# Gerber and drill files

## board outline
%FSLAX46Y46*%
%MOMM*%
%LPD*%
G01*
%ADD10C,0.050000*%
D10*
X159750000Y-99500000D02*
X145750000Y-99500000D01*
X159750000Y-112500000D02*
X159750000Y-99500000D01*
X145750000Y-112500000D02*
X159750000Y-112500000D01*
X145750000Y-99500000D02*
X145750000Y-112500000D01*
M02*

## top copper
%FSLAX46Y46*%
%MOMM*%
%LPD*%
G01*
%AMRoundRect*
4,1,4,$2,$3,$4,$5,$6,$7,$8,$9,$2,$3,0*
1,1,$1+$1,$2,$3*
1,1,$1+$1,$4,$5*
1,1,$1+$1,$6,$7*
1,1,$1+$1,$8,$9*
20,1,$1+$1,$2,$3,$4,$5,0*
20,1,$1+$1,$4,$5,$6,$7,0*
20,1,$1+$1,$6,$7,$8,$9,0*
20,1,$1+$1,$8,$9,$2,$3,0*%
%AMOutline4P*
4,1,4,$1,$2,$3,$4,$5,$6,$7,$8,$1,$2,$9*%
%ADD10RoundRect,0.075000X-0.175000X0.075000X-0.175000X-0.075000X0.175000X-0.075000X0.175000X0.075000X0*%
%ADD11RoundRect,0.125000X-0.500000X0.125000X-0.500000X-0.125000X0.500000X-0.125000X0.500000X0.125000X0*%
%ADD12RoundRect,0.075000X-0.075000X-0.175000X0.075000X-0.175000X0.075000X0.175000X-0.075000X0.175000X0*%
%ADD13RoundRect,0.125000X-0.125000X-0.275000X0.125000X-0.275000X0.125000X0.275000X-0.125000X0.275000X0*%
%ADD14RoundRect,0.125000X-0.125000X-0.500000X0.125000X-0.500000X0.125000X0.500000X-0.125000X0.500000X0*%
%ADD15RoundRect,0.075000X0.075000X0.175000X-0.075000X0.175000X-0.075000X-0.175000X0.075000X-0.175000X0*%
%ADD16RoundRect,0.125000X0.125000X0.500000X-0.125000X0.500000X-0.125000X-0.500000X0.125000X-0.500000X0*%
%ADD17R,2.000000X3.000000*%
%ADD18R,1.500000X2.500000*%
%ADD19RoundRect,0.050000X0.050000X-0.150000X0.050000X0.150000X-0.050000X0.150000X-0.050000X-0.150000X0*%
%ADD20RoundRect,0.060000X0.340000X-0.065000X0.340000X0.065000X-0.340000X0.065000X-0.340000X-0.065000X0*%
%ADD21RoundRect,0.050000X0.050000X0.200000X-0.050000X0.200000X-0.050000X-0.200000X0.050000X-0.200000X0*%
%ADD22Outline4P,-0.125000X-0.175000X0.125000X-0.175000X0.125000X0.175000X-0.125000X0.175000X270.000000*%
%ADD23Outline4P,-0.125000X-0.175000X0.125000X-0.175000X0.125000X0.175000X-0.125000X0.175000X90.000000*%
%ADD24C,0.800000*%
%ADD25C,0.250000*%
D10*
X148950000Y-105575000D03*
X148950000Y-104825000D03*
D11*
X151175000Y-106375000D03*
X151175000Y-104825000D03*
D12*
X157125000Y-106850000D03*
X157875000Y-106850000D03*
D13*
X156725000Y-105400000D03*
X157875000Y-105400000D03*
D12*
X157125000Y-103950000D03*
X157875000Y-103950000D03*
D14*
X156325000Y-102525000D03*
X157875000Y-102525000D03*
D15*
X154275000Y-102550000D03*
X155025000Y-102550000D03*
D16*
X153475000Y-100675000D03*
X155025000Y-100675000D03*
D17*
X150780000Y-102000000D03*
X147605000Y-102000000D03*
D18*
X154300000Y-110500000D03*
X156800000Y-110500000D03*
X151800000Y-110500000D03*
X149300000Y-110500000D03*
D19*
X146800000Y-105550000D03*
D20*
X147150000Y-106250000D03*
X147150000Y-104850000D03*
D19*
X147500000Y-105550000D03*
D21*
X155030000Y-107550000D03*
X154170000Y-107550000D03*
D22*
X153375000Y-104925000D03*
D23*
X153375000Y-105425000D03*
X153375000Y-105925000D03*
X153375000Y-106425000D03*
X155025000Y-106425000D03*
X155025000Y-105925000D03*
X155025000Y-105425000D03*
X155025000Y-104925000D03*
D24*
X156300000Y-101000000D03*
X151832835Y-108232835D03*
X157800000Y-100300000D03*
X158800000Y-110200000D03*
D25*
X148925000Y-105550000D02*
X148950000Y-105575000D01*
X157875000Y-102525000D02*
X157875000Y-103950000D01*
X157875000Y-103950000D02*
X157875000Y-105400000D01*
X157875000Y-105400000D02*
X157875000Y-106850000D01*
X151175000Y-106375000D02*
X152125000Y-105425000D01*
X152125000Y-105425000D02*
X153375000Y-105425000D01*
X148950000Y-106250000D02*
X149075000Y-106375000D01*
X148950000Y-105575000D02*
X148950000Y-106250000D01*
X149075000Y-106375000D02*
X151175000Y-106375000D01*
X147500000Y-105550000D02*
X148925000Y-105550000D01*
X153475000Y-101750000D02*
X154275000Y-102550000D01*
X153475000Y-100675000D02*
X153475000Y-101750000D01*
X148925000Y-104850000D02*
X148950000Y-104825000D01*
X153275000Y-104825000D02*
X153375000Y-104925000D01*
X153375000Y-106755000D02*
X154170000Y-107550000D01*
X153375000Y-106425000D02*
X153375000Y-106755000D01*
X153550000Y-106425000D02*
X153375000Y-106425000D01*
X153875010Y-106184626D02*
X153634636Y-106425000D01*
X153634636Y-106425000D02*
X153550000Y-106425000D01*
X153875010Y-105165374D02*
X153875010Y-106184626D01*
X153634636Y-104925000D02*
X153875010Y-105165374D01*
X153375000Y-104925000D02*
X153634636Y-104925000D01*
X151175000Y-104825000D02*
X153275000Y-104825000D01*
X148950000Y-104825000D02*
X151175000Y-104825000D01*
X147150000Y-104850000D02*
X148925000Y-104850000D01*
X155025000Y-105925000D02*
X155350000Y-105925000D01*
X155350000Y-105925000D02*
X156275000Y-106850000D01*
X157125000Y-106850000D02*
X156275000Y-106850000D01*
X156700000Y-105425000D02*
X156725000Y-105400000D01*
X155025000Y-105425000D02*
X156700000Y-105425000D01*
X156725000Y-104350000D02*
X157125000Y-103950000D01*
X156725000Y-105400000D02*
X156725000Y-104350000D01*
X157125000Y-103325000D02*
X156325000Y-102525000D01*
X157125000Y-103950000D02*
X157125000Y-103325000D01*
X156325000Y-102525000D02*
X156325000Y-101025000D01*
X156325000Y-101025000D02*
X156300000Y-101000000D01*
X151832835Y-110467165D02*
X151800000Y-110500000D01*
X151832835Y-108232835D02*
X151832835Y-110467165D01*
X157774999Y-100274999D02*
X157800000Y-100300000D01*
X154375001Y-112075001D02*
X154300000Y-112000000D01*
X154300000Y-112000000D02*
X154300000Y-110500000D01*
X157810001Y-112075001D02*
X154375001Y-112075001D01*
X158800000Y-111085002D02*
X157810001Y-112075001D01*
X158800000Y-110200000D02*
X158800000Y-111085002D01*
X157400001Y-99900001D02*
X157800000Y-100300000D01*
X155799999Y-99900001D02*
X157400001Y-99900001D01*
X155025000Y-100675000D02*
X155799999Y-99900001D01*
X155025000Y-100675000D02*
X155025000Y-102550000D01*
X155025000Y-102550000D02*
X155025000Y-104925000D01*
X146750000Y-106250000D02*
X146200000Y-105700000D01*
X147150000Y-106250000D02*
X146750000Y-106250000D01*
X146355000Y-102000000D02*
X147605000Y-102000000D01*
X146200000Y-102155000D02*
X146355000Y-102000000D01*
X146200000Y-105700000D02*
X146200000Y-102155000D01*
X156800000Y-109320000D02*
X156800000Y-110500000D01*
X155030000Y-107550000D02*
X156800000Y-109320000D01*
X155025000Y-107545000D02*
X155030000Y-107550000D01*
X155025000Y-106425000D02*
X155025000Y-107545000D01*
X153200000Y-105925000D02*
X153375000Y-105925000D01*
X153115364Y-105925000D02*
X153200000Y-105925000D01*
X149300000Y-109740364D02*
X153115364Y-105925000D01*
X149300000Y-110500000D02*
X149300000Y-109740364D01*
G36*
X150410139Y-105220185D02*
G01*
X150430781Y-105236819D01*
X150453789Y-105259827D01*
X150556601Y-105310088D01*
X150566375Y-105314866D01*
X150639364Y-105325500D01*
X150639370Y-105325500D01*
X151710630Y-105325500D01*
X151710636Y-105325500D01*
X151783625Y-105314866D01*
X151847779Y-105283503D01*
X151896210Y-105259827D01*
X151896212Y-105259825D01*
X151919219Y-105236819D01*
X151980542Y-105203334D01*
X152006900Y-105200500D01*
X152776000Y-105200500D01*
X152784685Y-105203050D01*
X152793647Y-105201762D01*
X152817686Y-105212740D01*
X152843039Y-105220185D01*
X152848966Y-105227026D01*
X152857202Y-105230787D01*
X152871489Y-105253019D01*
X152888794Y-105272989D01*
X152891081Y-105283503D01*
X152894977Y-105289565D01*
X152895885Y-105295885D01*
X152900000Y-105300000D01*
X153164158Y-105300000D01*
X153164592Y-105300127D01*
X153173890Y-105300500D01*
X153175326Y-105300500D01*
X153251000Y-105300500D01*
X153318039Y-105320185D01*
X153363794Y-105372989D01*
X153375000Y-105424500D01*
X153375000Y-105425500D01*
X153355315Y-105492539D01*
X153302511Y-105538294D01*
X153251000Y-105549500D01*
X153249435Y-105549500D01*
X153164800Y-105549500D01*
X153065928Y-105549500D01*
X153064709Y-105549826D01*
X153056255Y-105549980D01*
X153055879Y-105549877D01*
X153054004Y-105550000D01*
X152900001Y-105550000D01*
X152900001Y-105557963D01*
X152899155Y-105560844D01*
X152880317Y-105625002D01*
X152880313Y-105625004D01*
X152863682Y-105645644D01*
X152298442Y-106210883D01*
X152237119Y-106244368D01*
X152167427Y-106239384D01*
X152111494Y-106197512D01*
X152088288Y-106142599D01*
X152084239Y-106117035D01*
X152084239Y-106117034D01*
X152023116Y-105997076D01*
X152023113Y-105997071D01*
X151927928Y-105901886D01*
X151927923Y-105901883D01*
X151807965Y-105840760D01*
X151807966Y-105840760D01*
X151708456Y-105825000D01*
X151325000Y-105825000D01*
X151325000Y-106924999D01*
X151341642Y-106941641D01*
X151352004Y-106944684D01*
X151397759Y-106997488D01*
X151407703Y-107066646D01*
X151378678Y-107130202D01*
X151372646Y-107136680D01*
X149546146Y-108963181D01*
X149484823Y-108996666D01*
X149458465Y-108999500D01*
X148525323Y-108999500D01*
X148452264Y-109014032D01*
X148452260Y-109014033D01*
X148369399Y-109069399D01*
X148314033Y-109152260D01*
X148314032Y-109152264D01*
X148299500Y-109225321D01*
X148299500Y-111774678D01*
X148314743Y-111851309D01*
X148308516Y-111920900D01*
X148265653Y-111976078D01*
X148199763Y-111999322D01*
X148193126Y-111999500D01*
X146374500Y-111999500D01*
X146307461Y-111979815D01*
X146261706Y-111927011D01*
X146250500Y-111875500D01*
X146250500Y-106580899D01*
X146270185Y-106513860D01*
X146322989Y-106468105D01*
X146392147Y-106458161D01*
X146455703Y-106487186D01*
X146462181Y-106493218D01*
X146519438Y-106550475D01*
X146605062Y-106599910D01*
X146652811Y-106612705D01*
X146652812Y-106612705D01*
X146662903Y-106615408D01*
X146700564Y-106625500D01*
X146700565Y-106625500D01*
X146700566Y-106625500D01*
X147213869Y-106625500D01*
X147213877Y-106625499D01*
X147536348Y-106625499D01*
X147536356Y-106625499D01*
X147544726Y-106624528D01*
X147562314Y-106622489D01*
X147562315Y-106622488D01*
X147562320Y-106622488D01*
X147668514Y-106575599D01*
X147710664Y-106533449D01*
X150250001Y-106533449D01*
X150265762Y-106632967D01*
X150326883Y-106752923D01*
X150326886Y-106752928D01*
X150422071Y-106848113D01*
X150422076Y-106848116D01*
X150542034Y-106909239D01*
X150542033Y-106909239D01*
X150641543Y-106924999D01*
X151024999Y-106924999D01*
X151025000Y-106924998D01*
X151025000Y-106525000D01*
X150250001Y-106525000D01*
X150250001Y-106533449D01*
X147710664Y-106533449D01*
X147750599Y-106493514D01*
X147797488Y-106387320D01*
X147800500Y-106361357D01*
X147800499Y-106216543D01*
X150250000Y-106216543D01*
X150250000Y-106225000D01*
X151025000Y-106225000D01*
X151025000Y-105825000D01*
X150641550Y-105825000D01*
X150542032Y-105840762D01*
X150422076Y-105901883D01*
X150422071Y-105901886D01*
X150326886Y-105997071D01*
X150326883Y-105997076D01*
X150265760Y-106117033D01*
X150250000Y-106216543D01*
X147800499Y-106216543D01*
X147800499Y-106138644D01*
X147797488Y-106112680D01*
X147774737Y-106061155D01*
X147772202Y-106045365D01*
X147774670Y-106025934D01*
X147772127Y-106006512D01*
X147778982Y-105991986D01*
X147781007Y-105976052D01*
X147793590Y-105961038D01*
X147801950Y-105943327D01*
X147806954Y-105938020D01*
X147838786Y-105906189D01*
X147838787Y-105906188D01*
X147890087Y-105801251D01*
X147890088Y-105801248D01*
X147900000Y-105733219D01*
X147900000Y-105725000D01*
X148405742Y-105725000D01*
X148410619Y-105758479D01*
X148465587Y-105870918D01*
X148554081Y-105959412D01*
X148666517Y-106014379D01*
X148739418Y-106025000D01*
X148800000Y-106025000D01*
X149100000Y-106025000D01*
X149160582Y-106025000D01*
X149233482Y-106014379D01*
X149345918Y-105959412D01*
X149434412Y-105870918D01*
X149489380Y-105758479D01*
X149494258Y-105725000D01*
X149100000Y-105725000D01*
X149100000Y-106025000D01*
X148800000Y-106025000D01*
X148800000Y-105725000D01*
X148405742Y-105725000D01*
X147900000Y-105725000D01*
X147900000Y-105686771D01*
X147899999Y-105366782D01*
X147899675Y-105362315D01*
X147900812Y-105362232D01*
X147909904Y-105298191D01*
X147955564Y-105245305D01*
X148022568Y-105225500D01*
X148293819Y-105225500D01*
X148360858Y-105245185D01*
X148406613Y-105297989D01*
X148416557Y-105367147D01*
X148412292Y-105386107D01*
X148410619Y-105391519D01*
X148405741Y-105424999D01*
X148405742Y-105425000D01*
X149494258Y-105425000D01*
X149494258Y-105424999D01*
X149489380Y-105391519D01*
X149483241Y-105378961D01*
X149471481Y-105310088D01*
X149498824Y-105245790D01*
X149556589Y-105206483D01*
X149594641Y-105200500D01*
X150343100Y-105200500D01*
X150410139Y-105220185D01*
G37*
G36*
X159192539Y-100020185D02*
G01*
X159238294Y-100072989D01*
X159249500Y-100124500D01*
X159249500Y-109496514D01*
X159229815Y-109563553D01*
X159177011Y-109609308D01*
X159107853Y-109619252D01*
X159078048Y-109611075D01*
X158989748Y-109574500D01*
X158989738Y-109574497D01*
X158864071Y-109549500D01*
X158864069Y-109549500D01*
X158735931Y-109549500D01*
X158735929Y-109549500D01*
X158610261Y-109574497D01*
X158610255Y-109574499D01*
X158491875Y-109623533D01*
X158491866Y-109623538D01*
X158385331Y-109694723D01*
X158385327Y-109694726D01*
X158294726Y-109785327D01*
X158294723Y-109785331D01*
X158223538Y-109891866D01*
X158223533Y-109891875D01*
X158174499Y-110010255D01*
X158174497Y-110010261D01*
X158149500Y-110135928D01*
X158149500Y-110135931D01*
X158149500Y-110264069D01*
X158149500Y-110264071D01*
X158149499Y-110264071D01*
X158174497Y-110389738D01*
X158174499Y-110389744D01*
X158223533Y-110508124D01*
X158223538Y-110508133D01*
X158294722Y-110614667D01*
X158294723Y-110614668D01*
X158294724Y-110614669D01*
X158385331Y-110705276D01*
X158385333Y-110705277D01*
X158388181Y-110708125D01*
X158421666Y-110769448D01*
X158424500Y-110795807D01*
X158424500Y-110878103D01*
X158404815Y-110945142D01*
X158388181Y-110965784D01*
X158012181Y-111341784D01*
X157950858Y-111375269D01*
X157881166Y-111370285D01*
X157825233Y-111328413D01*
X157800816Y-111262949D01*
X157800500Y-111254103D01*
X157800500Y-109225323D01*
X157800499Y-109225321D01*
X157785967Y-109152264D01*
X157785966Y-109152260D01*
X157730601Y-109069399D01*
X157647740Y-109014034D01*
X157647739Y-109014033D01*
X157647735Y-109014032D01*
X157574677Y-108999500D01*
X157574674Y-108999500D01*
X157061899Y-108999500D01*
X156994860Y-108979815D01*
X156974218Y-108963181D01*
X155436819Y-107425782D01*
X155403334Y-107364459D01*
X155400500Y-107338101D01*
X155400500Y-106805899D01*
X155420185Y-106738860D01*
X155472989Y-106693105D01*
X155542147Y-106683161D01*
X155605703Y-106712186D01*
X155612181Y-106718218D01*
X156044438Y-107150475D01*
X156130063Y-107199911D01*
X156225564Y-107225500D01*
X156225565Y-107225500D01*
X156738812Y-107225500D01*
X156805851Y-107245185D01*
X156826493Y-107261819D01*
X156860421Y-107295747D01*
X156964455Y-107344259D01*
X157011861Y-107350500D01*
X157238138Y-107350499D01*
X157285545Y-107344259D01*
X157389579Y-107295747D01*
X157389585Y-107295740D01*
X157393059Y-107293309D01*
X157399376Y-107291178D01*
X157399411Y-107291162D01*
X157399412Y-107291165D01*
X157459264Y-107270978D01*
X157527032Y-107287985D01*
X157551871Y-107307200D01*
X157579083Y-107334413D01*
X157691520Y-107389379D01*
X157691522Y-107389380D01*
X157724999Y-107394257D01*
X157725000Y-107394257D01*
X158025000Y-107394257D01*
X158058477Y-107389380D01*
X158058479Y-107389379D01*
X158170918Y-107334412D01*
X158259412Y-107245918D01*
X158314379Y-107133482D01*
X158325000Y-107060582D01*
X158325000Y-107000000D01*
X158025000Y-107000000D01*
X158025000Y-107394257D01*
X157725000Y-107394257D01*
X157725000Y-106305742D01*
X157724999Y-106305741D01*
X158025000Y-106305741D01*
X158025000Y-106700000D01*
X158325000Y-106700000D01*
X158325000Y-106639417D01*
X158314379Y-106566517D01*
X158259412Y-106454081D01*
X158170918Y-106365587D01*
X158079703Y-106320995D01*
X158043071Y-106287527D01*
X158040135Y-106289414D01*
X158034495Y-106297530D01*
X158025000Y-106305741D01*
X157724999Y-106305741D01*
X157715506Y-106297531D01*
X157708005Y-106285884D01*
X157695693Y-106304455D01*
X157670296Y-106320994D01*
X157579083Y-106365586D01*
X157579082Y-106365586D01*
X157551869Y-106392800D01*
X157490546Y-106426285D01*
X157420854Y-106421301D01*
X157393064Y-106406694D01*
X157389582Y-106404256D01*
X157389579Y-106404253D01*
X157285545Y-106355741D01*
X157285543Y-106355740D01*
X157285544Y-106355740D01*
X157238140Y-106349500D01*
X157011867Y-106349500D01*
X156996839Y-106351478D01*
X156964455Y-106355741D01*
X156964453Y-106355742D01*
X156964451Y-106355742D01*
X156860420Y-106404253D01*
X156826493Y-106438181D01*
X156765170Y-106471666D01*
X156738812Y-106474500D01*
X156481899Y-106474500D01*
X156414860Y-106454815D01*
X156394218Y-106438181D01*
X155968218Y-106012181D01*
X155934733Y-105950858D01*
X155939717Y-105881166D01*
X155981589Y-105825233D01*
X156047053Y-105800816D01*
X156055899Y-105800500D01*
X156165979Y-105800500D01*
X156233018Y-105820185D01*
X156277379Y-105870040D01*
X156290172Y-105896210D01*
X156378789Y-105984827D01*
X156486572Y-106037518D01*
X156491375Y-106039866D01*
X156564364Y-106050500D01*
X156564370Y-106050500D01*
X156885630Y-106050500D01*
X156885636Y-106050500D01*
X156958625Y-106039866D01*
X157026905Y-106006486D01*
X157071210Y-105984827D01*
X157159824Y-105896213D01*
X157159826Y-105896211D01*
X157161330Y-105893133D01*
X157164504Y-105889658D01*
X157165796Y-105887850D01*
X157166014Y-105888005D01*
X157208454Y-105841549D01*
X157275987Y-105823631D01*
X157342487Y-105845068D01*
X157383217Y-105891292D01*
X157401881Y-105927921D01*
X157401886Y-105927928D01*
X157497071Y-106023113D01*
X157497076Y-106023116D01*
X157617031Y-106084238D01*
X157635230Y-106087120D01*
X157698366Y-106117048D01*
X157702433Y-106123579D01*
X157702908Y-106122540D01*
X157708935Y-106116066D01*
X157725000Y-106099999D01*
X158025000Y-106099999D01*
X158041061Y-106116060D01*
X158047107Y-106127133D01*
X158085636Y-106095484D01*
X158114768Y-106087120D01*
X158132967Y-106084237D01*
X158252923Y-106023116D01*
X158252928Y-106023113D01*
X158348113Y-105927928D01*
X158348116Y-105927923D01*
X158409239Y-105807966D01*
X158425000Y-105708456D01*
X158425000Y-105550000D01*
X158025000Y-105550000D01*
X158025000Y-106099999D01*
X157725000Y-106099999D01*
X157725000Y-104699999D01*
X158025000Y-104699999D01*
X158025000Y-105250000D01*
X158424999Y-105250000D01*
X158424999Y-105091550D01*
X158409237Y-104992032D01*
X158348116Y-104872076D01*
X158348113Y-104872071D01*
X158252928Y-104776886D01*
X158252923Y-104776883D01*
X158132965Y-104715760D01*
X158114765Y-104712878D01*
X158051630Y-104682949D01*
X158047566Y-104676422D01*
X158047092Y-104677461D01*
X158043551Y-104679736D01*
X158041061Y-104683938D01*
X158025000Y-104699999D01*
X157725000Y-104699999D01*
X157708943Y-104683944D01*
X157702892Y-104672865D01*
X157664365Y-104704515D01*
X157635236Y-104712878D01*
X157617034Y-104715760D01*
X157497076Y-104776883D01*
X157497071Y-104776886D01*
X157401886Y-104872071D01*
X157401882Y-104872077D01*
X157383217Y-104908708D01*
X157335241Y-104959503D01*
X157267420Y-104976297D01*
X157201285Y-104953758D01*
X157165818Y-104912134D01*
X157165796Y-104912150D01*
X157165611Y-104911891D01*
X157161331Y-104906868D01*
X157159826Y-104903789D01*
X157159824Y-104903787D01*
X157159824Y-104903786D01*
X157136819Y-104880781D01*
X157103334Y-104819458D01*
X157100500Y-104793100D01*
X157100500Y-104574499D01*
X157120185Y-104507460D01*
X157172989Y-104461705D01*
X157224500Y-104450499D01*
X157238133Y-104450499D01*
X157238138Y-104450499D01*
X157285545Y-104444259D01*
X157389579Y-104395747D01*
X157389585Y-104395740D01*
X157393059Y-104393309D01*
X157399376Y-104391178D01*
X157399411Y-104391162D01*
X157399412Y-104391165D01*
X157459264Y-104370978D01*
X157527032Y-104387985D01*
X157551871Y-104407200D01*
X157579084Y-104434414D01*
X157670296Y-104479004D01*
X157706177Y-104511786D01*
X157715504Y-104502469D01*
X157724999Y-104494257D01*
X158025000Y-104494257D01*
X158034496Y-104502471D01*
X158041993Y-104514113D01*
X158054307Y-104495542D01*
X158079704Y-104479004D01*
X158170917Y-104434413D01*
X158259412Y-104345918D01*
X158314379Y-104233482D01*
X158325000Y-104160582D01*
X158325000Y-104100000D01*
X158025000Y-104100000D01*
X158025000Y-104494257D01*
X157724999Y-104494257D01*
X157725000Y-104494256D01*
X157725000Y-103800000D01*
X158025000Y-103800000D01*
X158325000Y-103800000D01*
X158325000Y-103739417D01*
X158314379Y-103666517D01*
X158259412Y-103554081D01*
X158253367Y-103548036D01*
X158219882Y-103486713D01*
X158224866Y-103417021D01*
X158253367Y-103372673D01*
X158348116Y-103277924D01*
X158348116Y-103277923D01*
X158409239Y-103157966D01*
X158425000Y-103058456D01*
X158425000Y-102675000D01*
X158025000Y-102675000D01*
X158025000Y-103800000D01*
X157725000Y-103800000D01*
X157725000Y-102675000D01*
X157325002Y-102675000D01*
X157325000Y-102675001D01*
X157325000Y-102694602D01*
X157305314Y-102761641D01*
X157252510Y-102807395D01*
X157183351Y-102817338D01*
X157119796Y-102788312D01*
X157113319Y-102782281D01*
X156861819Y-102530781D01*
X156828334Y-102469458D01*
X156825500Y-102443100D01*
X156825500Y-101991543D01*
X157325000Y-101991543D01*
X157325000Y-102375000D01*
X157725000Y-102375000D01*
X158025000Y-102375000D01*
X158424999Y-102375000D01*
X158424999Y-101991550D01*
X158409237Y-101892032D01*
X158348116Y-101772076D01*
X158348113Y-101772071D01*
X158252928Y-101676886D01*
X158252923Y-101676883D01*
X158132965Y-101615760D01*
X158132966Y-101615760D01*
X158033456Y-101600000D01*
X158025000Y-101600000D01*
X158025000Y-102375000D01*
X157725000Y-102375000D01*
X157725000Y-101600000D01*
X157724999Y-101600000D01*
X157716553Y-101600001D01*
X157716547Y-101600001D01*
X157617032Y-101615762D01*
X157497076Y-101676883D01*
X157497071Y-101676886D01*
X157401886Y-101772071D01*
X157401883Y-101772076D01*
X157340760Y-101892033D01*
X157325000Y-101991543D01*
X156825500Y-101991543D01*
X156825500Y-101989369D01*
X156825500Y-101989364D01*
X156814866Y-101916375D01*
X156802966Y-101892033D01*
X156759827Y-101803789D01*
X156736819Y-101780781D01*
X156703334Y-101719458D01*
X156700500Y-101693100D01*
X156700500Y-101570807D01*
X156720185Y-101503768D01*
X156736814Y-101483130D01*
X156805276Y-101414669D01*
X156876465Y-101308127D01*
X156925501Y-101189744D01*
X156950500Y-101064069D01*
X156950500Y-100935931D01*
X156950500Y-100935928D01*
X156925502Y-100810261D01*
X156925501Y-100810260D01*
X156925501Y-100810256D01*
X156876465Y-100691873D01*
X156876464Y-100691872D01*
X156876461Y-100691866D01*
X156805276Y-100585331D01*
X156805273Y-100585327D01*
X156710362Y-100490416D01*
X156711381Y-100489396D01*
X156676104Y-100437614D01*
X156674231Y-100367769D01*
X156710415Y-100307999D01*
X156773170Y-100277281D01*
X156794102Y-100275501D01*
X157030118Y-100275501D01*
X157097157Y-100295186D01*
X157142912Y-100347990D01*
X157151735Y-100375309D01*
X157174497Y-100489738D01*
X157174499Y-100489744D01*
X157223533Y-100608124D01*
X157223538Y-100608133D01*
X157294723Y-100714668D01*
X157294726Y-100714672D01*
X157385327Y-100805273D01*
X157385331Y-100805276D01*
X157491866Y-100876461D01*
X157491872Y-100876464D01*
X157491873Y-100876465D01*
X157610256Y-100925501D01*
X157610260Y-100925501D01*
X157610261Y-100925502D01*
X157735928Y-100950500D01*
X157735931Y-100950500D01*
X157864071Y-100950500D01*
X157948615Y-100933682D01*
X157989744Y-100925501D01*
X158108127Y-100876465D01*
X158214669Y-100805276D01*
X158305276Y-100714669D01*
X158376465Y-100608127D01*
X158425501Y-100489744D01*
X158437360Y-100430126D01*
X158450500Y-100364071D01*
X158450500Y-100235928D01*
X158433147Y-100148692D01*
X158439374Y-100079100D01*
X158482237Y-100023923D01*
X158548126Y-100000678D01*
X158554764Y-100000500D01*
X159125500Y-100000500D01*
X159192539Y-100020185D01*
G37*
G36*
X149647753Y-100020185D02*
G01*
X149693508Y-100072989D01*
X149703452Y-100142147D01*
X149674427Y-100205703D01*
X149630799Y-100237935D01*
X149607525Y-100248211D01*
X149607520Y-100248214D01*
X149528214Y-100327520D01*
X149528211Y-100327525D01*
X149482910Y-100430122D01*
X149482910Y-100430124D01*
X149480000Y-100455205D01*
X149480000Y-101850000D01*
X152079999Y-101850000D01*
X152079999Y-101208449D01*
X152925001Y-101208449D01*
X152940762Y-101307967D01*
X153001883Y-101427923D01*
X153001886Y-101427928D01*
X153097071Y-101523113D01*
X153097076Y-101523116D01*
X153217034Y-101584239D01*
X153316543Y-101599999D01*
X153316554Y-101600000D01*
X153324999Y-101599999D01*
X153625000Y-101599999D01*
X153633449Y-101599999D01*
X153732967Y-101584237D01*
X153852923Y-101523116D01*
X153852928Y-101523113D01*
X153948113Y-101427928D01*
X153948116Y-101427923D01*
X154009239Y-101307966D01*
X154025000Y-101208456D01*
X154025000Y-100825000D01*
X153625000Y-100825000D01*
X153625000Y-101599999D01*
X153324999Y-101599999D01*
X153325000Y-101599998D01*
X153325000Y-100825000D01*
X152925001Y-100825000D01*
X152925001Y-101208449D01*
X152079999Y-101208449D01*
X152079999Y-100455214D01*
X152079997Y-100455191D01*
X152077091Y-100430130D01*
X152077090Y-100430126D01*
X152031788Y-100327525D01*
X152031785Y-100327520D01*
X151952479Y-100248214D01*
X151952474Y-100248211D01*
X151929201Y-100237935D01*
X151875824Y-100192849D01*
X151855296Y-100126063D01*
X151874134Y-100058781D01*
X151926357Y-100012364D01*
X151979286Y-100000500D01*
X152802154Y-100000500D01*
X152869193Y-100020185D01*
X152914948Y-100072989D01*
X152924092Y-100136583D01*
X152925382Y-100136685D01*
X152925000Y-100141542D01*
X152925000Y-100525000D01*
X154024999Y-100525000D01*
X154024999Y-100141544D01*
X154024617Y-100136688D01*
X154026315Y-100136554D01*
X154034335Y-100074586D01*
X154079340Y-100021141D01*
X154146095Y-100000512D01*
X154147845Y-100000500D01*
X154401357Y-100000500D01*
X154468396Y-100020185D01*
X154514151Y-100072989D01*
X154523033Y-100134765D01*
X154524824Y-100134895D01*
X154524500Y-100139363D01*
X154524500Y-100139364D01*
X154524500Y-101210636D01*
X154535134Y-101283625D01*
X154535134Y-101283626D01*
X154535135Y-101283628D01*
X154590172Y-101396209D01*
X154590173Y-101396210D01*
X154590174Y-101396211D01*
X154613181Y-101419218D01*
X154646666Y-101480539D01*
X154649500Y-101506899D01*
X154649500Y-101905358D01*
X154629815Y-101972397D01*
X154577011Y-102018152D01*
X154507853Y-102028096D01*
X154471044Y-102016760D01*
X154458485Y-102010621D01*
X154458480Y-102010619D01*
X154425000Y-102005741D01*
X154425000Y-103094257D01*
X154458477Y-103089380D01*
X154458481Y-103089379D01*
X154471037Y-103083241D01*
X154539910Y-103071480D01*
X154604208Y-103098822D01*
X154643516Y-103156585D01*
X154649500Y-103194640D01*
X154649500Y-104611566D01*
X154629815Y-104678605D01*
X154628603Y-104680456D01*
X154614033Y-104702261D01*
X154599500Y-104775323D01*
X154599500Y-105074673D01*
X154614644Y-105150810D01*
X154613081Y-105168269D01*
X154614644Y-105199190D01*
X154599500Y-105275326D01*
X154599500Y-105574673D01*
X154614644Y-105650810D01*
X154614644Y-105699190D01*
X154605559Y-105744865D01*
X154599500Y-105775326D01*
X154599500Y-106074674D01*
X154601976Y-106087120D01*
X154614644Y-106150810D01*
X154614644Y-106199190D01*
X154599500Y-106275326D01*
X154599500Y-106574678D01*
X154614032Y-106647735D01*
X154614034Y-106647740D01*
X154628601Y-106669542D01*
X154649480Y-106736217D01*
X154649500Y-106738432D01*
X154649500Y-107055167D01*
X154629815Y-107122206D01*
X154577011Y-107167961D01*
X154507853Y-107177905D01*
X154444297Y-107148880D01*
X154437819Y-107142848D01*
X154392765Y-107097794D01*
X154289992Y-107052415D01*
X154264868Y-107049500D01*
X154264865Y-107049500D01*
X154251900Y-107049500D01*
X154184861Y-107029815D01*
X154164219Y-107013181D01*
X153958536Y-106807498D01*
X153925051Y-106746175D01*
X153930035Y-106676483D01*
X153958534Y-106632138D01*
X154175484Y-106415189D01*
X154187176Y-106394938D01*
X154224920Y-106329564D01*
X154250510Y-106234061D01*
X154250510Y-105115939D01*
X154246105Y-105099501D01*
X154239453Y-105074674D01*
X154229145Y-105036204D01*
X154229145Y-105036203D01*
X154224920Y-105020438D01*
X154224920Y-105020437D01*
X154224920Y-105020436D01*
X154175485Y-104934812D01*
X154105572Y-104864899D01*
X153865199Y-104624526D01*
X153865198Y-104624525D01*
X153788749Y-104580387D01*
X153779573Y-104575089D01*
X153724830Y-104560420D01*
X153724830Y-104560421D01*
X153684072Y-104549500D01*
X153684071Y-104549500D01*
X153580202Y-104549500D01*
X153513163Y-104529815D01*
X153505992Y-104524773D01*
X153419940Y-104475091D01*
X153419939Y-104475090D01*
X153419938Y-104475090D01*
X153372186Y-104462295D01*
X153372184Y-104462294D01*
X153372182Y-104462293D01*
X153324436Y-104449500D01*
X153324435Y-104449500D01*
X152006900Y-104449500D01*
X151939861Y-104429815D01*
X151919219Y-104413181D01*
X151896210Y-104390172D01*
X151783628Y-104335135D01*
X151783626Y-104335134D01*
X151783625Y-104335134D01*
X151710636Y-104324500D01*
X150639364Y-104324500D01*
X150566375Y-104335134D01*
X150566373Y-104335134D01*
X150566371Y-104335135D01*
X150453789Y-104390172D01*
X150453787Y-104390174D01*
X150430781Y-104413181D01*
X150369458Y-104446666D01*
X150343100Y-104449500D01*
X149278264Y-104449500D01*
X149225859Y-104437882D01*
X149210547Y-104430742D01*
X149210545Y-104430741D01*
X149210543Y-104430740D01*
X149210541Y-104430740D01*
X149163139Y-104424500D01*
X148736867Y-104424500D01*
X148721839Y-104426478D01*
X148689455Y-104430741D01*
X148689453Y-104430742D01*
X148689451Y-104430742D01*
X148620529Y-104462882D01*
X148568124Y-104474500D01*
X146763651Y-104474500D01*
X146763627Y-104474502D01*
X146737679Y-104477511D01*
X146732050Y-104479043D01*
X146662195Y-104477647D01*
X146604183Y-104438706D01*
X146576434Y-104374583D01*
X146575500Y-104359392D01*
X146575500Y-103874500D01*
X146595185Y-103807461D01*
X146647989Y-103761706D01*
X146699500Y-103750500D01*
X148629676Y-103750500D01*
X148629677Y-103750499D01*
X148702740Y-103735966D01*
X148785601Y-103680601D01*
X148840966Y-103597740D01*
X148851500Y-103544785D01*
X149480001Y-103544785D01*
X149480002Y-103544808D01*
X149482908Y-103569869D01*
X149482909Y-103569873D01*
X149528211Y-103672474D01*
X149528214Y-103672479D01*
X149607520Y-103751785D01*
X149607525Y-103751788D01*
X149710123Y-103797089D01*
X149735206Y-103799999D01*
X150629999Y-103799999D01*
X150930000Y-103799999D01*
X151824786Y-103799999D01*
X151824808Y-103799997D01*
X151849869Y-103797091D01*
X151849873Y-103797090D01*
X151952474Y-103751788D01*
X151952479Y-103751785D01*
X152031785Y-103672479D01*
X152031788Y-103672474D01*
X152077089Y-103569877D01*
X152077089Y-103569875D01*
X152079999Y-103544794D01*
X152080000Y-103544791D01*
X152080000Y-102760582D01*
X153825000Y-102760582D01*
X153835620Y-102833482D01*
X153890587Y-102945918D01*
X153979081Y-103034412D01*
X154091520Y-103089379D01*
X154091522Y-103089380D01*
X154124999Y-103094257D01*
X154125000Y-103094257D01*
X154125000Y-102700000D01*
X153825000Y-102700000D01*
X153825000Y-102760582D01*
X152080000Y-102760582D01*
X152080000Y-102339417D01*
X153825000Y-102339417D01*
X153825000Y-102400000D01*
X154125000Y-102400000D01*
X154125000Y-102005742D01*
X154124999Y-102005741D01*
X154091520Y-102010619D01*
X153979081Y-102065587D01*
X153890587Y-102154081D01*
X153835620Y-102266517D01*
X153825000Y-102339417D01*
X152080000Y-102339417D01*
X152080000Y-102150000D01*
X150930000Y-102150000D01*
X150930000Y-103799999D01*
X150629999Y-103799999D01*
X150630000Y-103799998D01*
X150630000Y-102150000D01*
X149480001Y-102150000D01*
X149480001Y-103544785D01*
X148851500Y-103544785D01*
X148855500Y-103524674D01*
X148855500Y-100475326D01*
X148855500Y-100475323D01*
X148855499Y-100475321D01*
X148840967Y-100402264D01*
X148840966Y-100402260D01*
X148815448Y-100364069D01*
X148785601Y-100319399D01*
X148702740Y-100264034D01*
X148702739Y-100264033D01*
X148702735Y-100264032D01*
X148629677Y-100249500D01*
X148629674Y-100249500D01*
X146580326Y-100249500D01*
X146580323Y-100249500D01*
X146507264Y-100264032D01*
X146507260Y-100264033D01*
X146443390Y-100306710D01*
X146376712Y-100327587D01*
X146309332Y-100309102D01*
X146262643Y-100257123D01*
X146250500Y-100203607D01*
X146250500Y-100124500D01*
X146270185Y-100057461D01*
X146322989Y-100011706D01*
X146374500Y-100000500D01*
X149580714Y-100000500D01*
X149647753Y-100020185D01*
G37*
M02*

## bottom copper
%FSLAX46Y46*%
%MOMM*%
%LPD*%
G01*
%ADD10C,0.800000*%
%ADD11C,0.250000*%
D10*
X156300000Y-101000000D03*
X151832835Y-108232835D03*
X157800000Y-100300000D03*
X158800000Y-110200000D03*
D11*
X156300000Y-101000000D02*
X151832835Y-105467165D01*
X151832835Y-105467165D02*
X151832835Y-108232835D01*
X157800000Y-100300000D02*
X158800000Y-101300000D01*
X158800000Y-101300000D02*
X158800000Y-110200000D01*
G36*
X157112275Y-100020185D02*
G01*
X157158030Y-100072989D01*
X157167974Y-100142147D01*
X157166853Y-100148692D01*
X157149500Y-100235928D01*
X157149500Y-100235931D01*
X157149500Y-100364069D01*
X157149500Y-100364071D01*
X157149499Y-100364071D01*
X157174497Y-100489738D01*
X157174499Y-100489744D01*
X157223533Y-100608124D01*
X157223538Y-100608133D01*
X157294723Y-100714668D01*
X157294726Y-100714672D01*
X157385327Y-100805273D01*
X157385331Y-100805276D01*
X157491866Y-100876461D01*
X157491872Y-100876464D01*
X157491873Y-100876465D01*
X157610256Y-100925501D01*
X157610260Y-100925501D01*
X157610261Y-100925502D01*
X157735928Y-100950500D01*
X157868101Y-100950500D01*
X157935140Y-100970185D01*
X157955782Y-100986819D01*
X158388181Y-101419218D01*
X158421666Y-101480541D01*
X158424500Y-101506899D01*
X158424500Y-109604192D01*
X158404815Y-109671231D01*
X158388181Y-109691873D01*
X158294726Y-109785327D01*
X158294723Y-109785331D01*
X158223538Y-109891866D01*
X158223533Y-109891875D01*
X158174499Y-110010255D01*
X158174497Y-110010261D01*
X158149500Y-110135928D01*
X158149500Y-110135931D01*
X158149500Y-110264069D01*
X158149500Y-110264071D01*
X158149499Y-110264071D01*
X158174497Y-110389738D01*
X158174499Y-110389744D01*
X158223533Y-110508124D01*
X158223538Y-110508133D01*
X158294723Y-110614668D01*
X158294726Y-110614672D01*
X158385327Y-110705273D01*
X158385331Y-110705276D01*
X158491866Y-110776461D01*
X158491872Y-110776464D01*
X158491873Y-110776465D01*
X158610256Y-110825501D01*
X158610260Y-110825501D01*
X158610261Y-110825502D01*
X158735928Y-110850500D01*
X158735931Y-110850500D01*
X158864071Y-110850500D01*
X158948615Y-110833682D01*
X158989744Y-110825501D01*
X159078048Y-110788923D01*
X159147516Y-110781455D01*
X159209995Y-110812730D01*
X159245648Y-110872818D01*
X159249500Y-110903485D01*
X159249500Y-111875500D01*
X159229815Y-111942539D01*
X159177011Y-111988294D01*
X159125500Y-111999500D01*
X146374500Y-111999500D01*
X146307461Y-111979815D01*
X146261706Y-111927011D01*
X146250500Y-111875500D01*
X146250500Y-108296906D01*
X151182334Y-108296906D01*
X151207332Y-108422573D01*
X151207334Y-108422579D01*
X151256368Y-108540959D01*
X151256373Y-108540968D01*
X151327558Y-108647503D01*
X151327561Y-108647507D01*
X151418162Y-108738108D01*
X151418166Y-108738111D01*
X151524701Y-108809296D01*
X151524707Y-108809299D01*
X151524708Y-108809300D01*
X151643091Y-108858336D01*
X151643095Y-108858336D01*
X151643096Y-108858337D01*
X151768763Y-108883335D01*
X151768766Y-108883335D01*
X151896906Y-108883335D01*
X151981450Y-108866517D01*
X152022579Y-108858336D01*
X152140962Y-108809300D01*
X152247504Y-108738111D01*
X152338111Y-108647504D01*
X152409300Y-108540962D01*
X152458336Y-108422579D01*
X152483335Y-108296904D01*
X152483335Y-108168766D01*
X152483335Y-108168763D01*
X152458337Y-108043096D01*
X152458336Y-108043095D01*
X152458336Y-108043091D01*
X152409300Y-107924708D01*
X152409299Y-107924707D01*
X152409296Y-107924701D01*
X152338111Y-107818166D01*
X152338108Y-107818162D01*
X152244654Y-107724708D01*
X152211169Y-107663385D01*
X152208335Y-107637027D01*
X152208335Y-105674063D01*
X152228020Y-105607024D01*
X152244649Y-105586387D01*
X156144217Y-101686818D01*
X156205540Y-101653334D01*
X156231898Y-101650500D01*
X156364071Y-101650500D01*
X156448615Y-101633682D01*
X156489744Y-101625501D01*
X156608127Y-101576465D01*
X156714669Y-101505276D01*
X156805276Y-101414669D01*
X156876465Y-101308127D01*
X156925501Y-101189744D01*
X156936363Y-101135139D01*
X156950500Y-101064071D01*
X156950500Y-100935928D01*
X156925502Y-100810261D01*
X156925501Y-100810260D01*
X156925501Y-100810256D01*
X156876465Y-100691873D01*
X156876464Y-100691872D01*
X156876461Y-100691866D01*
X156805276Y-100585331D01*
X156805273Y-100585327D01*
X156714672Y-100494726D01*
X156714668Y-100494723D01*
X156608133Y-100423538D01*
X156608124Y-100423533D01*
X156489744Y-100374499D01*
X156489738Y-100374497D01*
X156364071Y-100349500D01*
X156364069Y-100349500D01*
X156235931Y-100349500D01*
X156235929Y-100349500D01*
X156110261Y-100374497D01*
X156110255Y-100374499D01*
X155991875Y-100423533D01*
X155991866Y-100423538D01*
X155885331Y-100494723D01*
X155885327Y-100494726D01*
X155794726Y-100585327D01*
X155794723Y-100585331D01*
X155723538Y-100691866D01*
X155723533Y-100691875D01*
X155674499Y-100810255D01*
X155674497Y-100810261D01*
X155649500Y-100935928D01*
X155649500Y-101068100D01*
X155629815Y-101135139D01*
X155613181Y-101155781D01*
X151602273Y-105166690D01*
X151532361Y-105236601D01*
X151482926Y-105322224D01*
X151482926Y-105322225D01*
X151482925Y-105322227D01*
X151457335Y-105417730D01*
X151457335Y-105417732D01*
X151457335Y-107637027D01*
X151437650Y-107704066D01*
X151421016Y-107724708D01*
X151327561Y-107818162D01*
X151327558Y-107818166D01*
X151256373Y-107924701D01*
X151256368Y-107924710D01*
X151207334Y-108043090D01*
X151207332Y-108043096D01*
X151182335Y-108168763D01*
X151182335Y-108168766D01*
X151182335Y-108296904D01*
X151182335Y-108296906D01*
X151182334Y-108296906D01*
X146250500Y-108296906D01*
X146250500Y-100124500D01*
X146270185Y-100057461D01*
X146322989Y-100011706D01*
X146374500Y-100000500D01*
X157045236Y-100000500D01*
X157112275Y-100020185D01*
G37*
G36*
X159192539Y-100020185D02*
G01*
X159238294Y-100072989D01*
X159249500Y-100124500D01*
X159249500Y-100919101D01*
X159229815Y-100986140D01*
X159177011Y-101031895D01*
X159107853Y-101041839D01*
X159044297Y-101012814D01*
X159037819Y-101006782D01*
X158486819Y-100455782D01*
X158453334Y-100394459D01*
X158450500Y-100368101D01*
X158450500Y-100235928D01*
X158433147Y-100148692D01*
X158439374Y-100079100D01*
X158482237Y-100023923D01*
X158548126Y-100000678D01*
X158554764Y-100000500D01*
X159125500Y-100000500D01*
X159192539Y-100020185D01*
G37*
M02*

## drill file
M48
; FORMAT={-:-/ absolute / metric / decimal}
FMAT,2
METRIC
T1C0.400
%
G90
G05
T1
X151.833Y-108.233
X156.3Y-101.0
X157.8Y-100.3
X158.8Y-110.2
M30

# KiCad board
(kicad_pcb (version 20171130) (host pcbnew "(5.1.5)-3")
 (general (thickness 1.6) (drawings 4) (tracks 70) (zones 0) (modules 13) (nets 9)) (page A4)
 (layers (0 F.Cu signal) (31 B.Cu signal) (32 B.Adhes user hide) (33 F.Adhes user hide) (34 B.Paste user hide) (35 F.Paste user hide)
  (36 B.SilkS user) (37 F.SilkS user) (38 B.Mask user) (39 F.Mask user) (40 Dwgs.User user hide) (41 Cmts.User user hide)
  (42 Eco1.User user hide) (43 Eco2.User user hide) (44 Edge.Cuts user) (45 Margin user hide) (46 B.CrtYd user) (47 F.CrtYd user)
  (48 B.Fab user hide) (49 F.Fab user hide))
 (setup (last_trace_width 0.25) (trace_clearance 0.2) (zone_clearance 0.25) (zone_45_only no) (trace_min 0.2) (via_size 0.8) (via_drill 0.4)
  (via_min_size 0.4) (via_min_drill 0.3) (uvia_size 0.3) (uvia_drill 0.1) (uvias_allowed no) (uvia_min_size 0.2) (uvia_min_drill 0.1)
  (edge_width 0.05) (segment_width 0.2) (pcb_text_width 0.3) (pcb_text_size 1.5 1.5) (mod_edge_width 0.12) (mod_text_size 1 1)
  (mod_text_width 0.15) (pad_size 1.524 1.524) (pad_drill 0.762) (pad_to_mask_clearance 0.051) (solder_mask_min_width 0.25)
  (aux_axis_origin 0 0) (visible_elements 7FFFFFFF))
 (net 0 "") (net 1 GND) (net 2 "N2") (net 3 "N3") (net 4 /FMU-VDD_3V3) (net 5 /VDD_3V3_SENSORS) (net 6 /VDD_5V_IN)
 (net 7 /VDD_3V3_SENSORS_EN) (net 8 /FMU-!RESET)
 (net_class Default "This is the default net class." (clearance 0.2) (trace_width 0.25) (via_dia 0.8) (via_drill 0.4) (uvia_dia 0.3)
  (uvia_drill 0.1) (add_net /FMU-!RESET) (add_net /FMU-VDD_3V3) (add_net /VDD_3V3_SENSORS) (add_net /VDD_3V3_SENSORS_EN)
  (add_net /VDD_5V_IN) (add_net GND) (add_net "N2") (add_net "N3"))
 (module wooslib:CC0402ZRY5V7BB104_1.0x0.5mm (layer F.Cu) (at 149.2 104.7 270)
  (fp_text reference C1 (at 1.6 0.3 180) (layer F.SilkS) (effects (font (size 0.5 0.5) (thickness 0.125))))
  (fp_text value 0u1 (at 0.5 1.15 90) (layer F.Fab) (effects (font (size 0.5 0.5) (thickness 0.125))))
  (pad 2 smd roundrect (at 0.875 0.25 270) (size 0.3 0.5) (layers F.Cu F.Paste F.Mask) (roundrect_rratio 0.25) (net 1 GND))
  (pad 1 smd roundrect (at 0.125 0.25 270) (size 0.3 0.5) (layers F.Cu F.Paste F.Mask) (roundrect_rratio 0.25) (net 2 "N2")))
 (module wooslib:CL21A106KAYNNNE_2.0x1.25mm (layer F.Cu) (at 151.8 104.6 270)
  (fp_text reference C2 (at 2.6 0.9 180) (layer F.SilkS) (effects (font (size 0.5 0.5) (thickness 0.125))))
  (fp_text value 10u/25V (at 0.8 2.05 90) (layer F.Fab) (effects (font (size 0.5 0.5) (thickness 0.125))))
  (pad 2 smd roundrect (at 1.775 0.625 270) (size 0.5 1.25) (layers F.Cu F.Paste F.Mask) (roundrect_rratio 0.25) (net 1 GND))
  (pad 1 smd roundrect (at 0.225 0.625 270) (size 0.5 1.25) (layers F.Cu F.Paste F.Mask) (roundrect_rratio 0.25) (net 2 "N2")))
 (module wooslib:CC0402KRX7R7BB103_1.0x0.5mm (layer F.Cu) (at 156.9 106.5)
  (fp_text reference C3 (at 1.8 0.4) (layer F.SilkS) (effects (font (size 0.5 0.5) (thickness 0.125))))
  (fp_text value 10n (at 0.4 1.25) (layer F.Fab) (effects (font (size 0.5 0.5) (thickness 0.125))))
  (pad 1 smd roundrect (at 0.225 0.35) (size 0.3 0.5) (layers F.Cu F.Paste F.Mask) (roundrect_rratio 0.25) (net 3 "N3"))
  (pad 2 smd roundrect (at 0.975 0.35) (size 0.3 0.5) (layers F.Cu F.Paste F.Mask) (roundrect_rratio 0.25) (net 1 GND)))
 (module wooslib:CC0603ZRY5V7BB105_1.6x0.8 (layer F.Cu) (at 156.5 105)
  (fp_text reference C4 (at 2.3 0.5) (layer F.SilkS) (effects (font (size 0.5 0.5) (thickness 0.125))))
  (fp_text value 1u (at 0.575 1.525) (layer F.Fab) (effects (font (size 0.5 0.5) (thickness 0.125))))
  (pad 1 smd roundrect (at 0.225 0.4) (size 0.5 0.8) (layers F.Cu F.Paste F.Mask) (roundrect_rratio 0.25) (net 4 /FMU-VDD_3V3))
  (pad 2 smd roundrect (at 1.375 0.4) (size 0.5 0.8) (layers F.Cu F.Paste F.Mask) (roundrect_rratio 0.25) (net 1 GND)))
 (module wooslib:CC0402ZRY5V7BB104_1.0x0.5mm (layer F.Cu) (at 157 103.7)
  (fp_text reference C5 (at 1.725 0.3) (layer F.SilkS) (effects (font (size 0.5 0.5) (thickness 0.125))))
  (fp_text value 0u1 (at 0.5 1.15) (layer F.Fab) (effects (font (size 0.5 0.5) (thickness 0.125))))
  (pad 1 smd roundrect (at 0.125 0.25) (size 0.3 0.5) (layers F.Cu F.Paste F.Mask) (roundrect_rratio 0.25) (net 4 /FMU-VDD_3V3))
  (pad 2 smd roundrect (at 0.875 0.25) (size 0.3 0.5) (layers F.Cu F.Paste F.Mask) (roundrect_rratio 0.25) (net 1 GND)))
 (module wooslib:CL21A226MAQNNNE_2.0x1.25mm (layer F.Cu) (at 156 101.8)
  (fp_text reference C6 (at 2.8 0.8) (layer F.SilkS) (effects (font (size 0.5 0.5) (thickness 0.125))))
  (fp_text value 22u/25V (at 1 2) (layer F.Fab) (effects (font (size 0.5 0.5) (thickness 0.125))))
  (pad 1 smd roundrect (at 0.325 0.725) (size 0.5 1.25) (layers F.Cu F.Paste F.Mask) (roundrect_rratio 0.25) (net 4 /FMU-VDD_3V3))
  (pad 2 smd roundrect (at 1.875 0.725) (size 0.5 1.25) (layers F.Cu F.Paste F.Mask) (roundrect_rratio 0.25) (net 1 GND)))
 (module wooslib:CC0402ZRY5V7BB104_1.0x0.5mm (layer F.Cu) (at 155.15 102.8 180)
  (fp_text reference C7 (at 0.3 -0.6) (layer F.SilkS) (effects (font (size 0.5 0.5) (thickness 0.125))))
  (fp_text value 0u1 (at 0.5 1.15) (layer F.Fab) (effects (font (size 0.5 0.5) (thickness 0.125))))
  (pad 2 smd roundrect (at 0.875 0.25 180) (size 0.3 0.5) (layers F.Cu F.Paste F.Mask) (roundrect_rratio 0.25) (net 1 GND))
  (pad 1 smd roundrect (at 0.125 0.25 180) (size 0.3 0.5) (layers F.Cu F.Paste F.Mask) (roundrect_rratio 0.25) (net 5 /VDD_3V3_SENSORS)))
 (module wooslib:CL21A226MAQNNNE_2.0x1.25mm (layer F.Cu) (at 155.35 101.4 180)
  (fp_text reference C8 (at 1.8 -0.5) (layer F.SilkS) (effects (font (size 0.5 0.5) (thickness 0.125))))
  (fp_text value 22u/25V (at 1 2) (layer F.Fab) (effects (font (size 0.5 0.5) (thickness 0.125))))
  (pad 2 smd roundrect (at 1.875 0.725 180) (size 0.5 1.25) (layers F.Cu F.Paste F.Mask) (roundrect_rratio 0.25) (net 1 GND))
  (pad 1 smd roundrect (at 0.325 0.725 180) (size 0.5 1.25) (layers F.Cu F.Paste F.Mask) (roundrect_rratio 0.25) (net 5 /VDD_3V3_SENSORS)))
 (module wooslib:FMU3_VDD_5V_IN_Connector (layer F.Cu) (at 145.7 102 90)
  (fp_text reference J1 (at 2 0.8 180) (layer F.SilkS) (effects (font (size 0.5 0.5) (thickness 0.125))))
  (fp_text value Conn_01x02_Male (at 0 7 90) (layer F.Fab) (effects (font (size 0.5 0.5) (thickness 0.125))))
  (pad 2 smd rect (at 0 5.08 90) (size 3 2) (layers F.Cu F.Paste F.Mask) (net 1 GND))
  (pad 1 smd rect (at 0 1.905 90) (size 3 2) (layers F.Cu F.Paste F.Mask) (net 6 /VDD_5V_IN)))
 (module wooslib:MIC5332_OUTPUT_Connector (layer F.Cu) (at 154.3 110.5 270)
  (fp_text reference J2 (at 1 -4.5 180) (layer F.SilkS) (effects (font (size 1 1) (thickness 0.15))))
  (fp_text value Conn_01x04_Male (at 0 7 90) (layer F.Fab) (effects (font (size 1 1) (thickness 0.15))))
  (pad 2 smd rect (at 0 0 270) (size 2.5 1.5) (layers F.Cu F.Paste F.Mask) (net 5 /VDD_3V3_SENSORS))
  (pad 1 smd rect (at 0 -2.5 270) (size 2.5 1.5) (layers F.Cu F.Paste F.Mask) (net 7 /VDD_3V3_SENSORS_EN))
  (pad 3 smd rect (at 0 2.5 270) (size 2.5 1.5) (layers F.Cu F.Paste F.Mask) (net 4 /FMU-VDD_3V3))
  (pad 4 smd rect (at 0 5 270) (size 2.5 1.5) (layers F.Cu F.Paste F.Mask) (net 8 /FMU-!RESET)))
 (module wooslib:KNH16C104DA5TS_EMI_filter (layer F.Cu) (at 146.8 106.3 90)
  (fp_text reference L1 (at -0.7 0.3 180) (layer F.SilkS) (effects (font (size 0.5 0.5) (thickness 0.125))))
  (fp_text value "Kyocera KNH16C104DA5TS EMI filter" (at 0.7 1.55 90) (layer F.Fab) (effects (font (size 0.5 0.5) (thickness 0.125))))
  (pad 4 smd roundrect (at 0.75 0 90) (size 0.4 0.2) (layers F.Cu F.Paste F.Mask) (roundrect_rratio 0.25))
  (pad 1 smd roundrect (at 0.05 0.35 90) (size 0.25 0.8) (layers F.Cu F.Paste F.Mask) (roundrect_rratio 0.24) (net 6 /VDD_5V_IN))
  (pad 3 smd roundrect (at 1.45 0.35 90) (size 0.25 0.8) (layers F.Cu F.Paste F.Mask) (roundrect_rratio 0.24) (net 2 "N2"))
  (pad 2 smd roundrect (at 0.75 0.7 90) (size 0.4 0.2) (layers F.Cu F.Paste F.Mask) (roundrect_rratio 0.25) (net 1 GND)))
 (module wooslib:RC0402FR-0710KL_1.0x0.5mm (layer F.Cu) (at 155.1 107.8 180)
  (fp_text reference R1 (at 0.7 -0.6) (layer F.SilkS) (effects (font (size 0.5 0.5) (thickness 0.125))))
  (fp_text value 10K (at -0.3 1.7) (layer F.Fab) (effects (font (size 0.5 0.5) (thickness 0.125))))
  (pad 1 smd roundrect (at 0.07 0.25 180) (size 0.2 0.5) (layers F.Cu F.Paste F.Mask) (roundrect_rratio 0.25) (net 7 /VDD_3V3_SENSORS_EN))
  (pad 2 smd roundrect (at 0.93 0.25 180) (size 0.2 0.5) (layers F.Cu F.Paste F.Mask) (roundrect_rratio 0.25) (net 2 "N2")))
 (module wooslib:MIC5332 (layer F.Cu) (at 153.2 104.8)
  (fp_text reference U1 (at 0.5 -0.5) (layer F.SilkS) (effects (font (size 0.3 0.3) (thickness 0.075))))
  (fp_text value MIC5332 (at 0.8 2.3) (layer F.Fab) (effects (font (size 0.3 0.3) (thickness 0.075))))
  (pad 1 smd trapezoid (at 0.175 0.125 270) (size 0.25 0.35) (layers F.Cu F.Paste F.Mask) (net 2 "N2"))
  (pad 2 smd trapezoid (at 0.175 0.625 90) (size 0.25 0.35) (layers F.Cu F.Paste F.Mask) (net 1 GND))
  (pad 3 smd trapezoid (at 0.175 1.125 90) (size 0.25 0.35) (layers F.Cu F.Paste F.Mask) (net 8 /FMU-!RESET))
  (pad 4 smd trapezoid (at 0.175 1.625 90) (size 0.25 0.35) (layers F.Cu F.Paste F.Mask) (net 2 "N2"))
  (pad 5 smd trapezoid (at 1.825 1.625 90) (size 0.25 0.35) (layers F.Cu F.Paste F.Mask) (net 7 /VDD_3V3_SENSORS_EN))
  (pad 6 smd trapezoid (at 1.825 1.125 90) (size 0.25 0.35) (layers F.Cu F.Paste F.Mask) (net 3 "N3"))
  (pad 7 smd trapezoid (at 1.825 0.625 90) (size 0.25 0.35) (layers F.Cu F.Paste F.Mask) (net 4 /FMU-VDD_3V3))
  (pad 8 smd trapezoid (at 1.825 0.125 90) (size 0.25 0.35) (layers F.Cu F.Paste F.Mask) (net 5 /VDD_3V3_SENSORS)))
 (gr_line (start 159.75 99.5) (end 145.75 99.5) (layer Edge.Cuts) (width 0.05))
 (gr_line (start 159.75 112.5) (end 159.75 99.5) (layer Edge.Cuts) (width 0.05))
 (gr_line (start 145.75 112.5) (end 159.75 112.5) (layer Edge.Cuts) (width 0.05))
 (gr_line (start 145.75 99.5) (end 145.75 112.5) (layer Edge.Cuts) (width 0.05))
 (segment (start 148.925 105.55) (end 148.95 105.575) (width 0.25) (layer F.Cu) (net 1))
 (segment (start 157.875 102.525) (end 157.875 103.95) (width 0.25) (layer F.Cu) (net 1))
 (segment (start 157.875 103.95) (end 157.875 105.4) (width 0.25) (layer F.Cu) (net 1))
 (segment (start 157.875 105.4) (end 157.875 106.85) (width 0.25) (layer F.Cu) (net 1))
 (segment (start 151.175 106.375) (end 152.125 105.425) (width 0.25) (layer F.Cu) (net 1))
 (segment (start 152.125 105.425) (end 153.375 105.425) (width 0.25) (layer F.Cu) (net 1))
 (segment (start 148.95 106.25) (end 149.075 106.375) (width 0.25) (layer F.Cu) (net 1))
 (segment (start 148.95 105.575) (end 148.95 106.25) (width 0.25) (layer F.Cu) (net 1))
 (segment (start 149.075 106.375) (end 151.175 106.375) (width 0.25) (layer F.Cu) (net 1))
 (segment (start 147.5 105.55) (end 148.925 105.55) (width 0.25) (layer F.Cu) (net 1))
 (segment (start 153.475 101.75) (end 154.275 102.55) (width 0.25) (layer F.Cu) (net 1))
 (segment (start 153.475 100.675) (end 153.475 101.75) (width 0.25) (layer F.Cu) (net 1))
 (segment (start 148.925 104.85) (end 148.95 104.825) (width 0.25) (layer F.Cu) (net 2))
 (segment (start 153.275 104.825) (end 153.375 104.925) (width 0.25) (layer F.Cu) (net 2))
 (segment (start 153.375 106.755) (end 154.17 107.55) (width 0.25) (layer F.Cu) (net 2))
 (segment (start 153.375 106.425) (end 153.375 106.755) (width 0.25) (layer F.Cu) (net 2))
 (segment (start 153.55 106.425) (end 153.375 106.425) (width 0.25) (layer F.Cu) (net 2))
 (segment (start 153.87501 106.184626) (end 153.634636 106.425) (width 0.25) (layer F.Cu) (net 2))
 (segment (start 153.634636 106.425) (end 153.55 106.425) (width 0.25) (layer F.Cu) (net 2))
 (segment (start 153.87501 105.165374) (end 153.87501 106.184626) (width 0.25) (layer F.Cu) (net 2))
 (segment (start 153.634636 104.925) (end 153.87501 105.165374) (width 0.25) (layer F.Cu) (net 2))
 (segment (start 153.375 104.925) (end 153.634636 104.925) (width 0.25) (layer F.Cu) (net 2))
 (segment (start 151.175 104.825) (end 153.275 104.825) (width 0.25) (layer F.Cu) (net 2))
 (segment (start 148.95 104.825) (end 151.175 104.825) (width 0.25) (layer F.Cu) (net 2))
 (segment (start 147.15 104.85) (end 148.925 104.85) (width 0.25) (layer F.Cu) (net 2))
 (segment (start 155.025 105.925) (end 155.35 105.925) (width 0.25) (layer F.Cu) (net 3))
 (segment (start 155.35 105.925) (end 156.275 106.85) (width 0.25) (layer F.Cu) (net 3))
 (segment (start 157.125 106.85) (end 156.275 106.85) (width 0.25) (layer F.Cu) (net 3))
 (segment (start 156.7 105.425) (end 156.725 105.4) (width 0.25) (layer F.Cu) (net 4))
 (segment (start 155.025 105.425) (end 156.7 105.425) (width 0.25) (layer F.Cu) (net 4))
 (segment (start 156.725 104.35) (end 157.125 103.95) (width 0.25) (layer F.Cu) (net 4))
 (segment (start 156.725 105.4) (end 156.725 104.35) (width 0.25) (layer F.Cu) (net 4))
 (segment (start 157.125 103.325) (end 156.325 102.525) (width 0.25) (layer F.Cu) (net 4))
 (segment (start 157.125 103.95) (end 157.125 103.325) (width 0.25) (layer F.Cu) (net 4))
 (via (at 156.3 101) (size 0.8) (drill 0.4) (layers F.Cu B.Cu) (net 4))
 (segment (start 156.325 102.525) (end 156.325 101.025) (width 0.25) (layer F.Cu) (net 4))
 (segment (start 156.325 101.025) (end 156.3 101) (width 0.25) (layer F.Cu) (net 4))
 (via (at 151.832835 108.232835) (size 0.8) (drill 0.4) (layers F.Cu B.Cu) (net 4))
 (segment (start 156.3 101) (end 151.832835 105.467165) (width 0.25) (layer B.Cu) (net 4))
 (segment (start 151.832835 105.467165) (end 151.832835 108.232835) (width 0.25) (layer B.Cu) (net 4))
 (segment (start 151.832835 110.467165) (end 151.8 110.5) (width 0.25) (layer F.Cu) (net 4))
 (segment (start 151.832835 108.232835) (end 151.832835 110.467165) (width 0.25) (layer F.Cu) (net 4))
 (via (at 157.8 100.3) (size 0.8) (drill 0.4) (layers F.Cu B.Cu) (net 5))
 (segment (start 157.774999 100.274999) (end 157.8 100.3) (width 0.25) (layer F.Cu) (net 5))
 (via (at 158.8 110.2) (size 0.8) (drill 0.4) (layers F.Cu B.Cu) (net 5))
 (segment (start 157.8 100.3) (end 158.8 101.3) (width 0.25) (layer B.Cu) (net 5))
 (segment (start 158.8 101.3) (end 158.8 110.2) (width 0.25) (layer B.Cu) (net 5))
 (segment (start 154.375001 112.075001) (end 154.3 112) (width 0.25) (layer F.Cu) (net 5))
 (segment (start 154.3 112) (end 154.3 110.5) (width 0.25) (layer F.Cu) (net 5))
 (segment (start 157.810001 112.075001) (end 154.375001 112.075001) (width 0.25) (layer F.Cu) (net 5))
 (segment (start 158.8 111.085002) (end 157.810001 112.075001) (width 0.25) (layer F.Cu) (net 5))
 (segment (start 158.8 110.2) (end 158.8 111.085002) (width 0.25) (layer F.Cu) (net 5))
 (segment (start 157.400001 99.900001) (end 157.8 100.3) (width 0.25) (layer F.Cu) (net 5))
 (segment (start 155.799999 99.900001) (end 157.400001 99.900001) (width 0.25) (layer F.Cu) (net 5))
 (segment (start 155.025 100.675) (end 155.799999 99.900001) (width 0.25) (layer F.Cu) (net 5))
 (segment (start 155.025 100.675) (end 155.025 102.55) (width 0.25) (layer F.Cu) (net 5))
 (segment (start 155.025 102.55) (end 155.025 104.925) (width 0.25) (layer F.Cu) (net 5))
 (segment (start 146.75 106.25) (end 146.2 105.7) (width 0.25) (layer F.Cu) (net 6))
 (segment (start 147.15 106.25) (end 146.75 106.25) (width 0.25) (layer F.Cu) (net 6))
 (segment (start 146.355 102) (end 147.605 102) (width 0.25) (layer F.Cu) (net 6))
 (segment (start 146.2 102.155) (end 146.355 102) (width 0.25) (layer F.Cu) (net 6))
 (segment (start 146.2 105.7) (end 146.2 102.155) (width 0.25) (layer F.Cu) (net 6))
 (segment (start 156.8 109.32) (end 156.8 110.5) (width 0.25) (layer F.Cu) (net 7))
 (segment (start 155.03 107.55) (end 156.8 109.32) (width 0.25) (layer F.Cu) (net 7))
 (segment (start 155.025 107.545) (end 155.03 107.55) (width 0.25) (layer F.Cu) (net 7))
 (segment (start 155.025 106.425) (end 155.025 107.545) (width 0.25) (layer F.Cu) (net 7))
 (segment (start 153.2 105.925) (end 153.375 105.925) (width 0.25) (layer F.Cu) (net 8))
 (segment (start 153.115364 105.925) (end 153.2 105.925) (width 0.25) (layer F.Cu) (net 8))
 (segment (start 149.3 109.740364) (end 153.115364 105.925) (width 0.25) (layer F.Cu) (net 8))
 (segment (start 149.3 110.5) (end 149.3 109.740364) (width 0.25) (layer F.Cu) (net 8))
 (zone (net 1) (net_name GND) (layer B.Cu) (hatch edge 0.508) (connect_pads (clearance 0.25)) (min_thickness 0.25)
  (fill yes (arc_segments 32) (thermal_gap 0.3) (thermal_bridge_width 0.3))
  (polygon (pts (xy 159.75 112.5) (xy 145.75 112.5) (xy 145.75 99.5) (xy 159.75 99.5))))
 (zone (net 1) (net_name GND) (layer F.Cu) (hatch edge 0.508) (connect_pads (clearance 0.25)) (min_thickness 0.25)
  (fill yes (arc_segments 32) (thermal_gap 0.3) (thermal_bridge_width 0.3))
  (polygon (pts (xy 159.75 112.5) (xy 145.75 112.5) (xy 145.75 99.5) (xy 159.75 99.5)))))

